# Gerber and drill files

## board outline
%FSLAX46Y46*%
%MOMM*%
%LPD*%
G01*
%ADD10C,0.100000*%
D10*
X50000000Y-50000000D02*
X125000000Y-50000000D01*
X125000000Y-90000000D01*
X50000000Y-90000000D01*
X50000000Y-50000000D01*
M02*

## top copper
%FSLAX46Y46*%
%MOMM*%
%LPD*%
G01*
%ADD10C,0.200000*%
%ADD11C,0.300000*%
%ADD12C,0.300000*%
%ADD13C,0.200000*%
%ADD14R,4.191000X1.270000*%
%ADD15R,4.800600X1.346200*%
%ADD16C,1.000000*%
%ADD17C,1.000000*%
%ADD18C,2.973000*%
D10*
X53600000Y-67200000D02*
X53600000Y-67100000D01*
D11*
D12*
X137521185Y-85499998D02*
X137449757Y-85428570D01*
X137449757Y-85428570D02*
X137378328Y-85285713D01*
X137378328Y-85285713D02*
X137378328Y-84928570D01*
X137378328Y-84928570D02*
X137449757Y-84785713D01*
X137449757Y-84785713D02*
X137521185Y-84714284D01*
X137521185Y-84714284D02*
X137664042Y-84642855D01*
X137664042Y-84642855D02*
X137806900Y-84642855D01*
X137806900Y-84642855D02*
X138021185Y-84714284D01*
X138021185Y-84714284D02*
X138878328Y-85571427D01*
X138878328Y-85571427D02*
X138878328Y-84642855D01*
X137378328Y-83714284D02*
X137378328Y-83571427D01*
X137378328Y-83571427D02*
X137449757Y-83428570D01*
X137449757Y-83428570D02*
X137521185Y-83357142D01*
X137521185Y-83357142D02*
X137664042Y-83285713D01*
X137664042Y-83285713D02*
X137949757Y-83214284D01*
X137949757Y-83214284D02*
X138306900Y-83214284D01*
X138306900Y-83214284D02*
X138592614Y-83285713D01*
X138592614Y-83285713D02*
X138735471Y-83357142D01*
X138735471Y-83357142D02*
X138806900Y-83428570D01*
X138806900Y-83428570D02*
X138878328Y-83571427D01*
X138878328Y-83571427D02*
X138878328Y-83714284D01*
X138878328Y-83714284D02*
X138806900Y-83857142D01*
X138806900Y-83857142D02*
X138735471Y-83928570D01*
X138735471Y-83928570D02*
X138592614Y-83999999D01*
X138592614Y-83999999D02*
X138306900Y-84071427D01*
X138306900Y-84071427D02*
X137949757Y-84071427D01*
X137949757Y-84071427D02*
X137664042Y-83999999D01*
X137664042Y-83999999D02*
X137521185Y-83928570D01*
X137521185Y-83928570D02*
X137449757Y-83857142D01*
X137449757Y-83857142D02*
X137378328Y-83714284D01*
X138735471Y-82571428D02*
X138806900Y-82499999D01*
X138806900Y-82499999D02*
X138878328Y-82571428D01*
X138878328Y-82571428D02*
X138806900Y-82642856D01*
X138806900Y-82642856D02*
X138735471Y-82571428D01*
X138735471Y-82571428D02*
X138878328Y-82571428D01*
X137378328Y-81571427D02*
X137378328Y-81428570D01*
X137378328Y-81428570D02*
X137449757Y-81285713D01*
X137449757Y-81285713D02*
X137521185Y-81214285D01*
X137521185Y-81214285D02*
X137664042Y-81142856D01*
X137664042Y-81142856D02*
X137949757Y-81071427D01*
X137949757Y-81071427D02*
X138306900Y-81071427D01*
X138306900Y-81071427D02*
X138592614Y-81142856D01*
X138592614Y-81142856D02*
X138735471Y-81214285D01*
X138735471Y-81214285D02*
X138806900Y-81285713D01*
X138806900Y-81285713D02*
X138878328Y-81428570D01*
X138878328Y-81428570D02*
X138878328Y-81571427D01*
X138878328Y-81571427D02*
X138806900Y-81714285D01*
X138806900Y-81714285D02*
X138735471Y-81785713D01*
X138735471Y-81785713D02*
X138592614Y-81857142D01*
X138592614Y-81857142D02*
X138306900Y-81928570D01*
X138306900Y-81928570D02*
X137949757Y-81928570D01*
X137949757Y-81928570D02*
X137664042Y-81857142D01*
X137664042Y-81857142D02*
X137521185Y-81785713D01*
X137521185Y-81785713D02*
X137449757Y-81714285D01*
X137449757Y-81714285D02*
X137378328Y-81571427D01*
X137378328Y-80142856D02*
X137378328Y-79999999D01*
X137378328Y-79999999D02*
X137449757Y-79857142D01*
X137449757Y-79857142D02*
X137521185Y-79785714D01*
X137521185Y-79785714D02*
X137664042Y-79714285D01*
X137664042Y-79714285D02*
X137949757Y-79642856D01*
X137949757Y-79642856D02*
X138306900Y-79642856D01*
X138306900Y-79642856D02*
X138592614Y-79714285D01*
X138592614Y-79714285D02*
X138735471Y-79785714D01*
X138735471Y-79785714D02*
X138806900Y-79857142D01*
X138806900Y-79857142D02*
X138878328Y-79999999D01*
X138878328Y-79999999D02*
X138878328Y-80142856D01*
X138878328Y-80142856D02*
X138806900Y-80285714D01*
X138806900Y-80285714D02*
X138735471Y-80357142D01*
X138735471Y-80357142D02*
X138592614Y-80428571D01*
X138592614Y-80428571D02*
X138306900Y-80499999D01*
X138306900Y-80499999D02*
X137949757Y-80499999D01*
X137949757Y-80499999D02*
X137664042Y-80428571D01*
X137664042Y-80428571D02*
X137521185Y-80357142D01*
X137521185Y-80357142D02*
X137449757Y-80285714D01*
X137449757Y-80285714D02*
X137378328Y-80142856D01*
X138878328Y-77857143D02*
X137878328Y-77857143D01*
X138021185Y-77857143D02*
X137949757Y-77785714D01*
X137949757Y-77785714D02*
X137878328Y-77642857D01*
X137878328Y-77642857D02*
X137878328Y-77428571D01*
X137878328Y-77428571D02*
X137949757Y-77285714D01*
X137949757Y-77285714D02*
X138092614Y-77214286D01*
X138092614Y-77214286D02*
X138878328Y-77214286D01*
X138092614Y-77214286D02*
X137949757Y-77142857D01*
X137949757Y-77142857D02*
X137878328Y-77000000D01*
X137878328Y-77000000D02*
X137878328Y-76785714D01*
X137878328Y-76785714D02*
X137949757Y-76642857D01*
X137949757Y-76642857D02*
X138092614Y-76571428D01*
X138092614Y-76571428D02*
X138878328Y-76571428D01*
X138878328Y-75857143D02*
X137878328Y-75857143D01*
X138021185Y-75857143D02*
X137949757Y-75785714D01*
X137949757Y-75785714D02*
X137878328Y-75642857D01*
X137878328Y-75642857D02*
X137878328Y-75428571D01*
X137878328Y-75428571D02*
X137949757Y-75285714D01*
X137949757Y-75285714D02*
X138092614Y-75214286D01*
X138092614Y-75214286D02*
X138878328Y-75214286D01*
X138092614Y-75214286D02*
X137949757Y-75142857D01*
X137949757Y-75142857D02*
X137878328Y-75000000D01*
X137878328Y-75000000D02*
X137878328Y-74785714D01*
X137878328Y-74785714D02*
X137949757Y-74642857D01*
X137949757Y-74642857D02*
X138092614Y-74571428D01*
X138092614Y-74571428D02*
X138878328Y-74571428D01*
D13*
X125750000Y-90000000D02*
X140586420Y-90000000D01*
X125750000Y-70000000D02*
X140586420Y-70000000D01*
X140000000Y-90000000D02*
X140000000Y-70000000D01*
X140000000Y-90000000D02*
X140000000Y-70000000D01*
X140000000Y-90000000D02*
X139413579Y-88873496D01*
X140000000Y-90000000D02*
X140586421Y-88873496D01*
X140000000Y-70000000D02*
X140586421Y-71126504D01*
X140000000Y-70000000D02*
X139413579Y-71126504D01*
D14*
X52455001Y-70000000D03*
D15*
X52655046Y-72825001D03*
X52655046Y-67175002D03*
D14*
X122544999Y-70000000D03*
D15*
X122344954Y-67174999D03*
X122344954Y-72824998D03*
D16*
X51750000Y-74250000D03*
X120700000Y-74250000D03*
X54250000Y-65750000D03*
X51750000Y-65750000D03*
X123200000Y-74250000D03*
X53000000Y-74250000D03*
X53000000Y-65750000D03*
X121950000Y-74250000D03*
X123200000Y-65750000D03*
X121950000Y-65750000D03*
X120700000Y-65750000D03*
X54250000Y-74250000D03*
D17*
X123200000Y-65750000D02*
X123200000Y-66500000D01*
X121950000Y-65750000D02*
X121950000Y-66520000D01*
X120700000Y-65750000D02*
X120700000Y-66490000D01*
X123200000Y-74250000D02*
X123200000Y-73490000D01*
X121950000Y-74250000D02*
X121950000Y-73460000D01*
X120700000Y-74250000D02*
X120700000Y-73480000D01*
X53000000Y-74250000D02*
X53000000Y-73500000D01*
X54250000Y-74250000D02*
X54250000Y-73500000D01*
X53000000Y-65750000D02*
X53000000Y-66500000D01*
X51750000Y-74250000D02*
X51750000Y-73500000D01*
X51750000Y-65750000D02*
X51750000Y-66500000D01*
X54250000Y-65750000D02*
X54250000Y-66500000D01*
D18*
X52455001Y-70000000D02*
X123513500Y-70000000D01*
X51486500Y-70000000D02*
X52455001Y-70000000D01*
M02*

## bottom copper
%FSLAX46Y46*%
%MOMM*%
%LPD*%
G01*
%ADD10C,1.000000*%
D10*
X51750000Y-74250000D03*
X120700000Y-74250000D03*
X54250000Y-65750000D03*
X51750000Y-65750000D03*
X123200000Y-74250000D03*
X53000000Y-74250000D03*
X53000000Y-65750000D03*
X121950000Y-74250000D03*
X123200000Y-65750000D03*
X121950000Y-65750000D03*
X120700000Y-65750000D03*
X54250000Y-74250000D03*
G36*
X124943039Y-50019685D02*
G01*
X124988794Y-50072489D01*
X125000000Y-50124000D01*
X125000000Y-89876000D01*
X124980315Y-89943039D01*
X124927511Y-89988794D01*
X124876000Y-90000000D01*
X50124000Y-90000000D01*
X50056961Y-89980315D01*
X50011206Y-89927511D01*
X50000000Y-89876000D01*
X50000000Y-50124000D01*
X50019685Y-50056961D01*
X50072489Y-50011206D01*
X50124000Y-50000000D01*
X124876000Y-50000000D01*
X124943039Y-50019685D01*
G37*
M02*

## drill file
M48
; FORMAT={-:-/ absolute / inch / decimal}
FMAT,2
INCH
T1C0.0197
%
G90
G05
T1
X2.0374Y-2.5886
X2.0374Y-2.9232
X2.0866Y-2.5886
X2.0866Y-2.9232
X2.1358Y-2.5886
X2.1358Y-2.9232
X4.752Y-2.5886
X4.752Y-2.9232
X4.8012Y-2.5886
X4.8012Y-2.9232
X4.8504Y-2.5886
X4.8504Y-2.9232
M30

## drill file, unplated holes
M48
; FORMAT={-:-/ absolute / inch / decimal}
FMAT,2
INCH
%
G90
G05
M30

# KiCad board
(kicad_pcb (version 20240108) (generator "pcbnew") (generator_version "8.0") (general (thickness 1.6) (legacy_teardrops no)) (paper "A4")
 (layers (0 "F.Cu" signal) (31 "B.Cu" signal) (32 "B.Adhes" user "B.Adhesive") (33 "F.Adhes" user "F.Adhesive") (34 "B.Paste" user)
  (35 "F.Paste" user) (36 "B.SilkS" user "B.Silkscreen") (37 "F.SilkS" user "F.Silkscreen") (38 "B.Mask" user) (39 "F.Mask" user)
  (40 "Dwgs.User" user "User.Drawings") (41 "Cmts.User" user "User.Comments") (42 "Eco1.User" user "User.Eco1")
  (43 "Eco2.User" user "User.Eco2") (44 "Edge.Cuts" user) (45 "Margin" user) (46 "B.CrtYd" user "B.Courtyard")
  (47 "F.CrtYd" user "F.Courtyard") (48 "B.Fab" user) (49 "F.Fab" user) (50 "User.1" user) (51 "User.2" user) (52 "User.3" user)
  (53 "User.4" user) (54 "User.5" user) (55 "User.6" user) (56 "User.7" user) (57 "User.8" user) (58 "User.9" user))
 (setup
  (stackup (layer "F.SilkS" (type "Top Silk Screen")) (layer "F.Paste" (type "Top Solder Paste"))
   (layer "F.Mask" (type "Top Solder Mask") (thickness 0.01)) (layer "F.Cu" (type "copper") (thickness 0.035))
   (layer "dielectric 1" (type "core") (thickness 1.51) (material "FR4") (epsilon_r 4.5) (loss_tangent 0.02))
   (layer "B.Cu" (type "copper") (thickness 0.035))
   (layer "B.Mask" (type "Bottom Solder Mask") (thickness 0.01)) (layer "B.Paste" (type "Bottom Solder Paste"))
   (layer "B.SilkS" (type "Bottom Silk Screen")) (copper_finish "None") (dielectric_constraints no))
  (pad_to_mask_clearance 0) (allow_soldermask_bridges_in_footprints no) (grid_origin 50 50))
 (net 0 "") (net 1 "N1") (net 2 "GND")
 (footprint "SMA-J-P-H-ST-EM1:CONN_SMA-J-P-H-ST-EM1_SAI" (layer "F.Cu") (at 52.16 70 90)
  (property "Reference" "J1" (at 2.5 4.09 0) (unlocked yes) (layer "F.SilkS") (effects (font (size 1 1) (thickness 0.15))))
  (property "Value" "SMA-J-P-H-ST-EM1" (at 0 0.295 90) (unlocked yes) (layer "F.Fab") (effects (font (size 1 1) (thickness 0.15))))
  (pad "1" smd rect (at 0 0.295001 90) (size 1.27 4.191) (layers "F.Cu" "F.Paste" "F.Mask") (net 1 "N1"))
  (pad "2" smd rect (at -2.825001 0.495046 90) (size 1.3462 4.8006) (layers "F.Cu" "F.Paste" "F.Mask") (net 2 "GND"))
  (pad "3" smd rect (at 2.824998 0.495046 90) (size 1.3462 4.8006) (layers "F.Cu" "F.Paste" "F.Mask") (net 2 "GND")))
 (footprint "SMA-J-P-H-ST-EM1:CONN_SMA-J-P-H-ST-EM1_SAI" (layer "F.Cu") (at 122.84 70 -90)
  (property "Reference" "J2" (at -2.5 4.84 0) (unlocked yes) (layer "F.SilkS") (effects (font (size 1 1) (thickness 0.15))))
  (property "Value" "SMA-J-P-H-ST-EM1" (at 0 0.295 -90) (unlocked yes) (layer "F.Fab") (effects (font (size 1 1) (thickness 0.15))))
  (pad "1" smd rect (at 0 0.295001 270) (size 1.27 4.191) (layers "F.Cu" "F.Paste" "F.Mask") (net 1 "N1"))
  (pad "2" smd rect (at -2.825001 0.495046 270) (size 1.3462 4.8006) (layers "F.Cu" "F.Paste" "F.Mask") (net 2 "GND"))
  (pad "3" smd rect (at 2.824998 0.495046 270) (size 1.3462 4.8006) (layers "F.Cu" "F.Paste" "F.Mask") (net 2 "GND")))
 (gr_line (start 53.6 67.2) (end 53.6 67.1) (stroke (width 0.2) (type default)) (layer "F.Cu") (net 2))
 (gr_rect (start 50 50) (end 125 90) (stroke (width 0.1) (type default)) (fill none) (layer "Edge.Cuts"))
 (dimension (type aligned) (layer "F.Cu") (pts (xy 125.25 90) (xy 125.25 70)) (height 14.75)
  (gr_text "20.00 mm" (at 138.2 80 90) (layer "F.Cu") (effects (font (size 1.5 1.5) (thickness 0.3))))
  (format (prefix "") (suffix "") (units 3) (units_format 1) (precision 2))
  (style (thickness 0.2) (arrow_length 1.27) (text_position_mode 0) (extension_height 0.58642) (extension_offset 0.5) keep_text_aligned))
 (segment (start 123.2 65.75) (end 123.2 66.5) (width 1) (layer "F.Cu") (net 2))
 (segment (start 120.7 74.25) (end 120.7 73.48) (width 1) (layer "F.Cu") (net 2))
 (segment (start 53 74.25) (end 53 73.5) (width 1) (layer "F.Cu") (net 2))
 (segment (start 54.25 74.25) (end 54.25 73.5) (width 1) (layer "F.Cu") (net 2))
 (segment (start 53 65.75) (end 53 66.5) (width 1) (layer "F.Cu") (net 2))
 (segment (start 123.2 74.25) (end 123.2 73.49) (width 1) (layer "F.Cu") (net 2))
 (segment (start 121.95 65.75) (end 121.95 66.52) (width 1) (layer "F.Cu") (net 2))
 (segment (start 51.75 74.25) (end 51.75 73.5) (width 1) (layer "F.Cu") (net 2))
 (segment (start 51.75 65.75) (end 51.75 66.5) (width 1) (layer "F.Cu") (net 2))
 (segment (start 54.25 65.75) (end 54.25 66.5) (width 1) (layer "F.Cu") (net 2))
 (segment (start 120.7 65.75) (end 120.7 66.49) (width 1) (layer "F.Cu") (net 2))
 (segment (start 121.95 74.25) (end 121.95 73.46) (width 1) (layer "F.Cu") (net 2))
 (via (at 51.75 74.25) (size 1) (drill 0.5) (layers "F.Cu" "B.Cu") (free yes) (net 2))
 (via (at 120.7 74.25) (size 1) (drill 0.5) (layers "F.Cu" "B.Cu") (free yes) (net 2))
 (via (at 54.25 65.75) (size 1) (drill 0.5) (layers "F.Cu" "B.Cu") (free yes) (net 2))
 (via (at 51.75 65.75) (size 1) (drill 0.5) (layers "F.Cu" "B.Cu") (free yes) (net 2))
 (via (at 123.2 74.25) (size 1) (drill 0.5) (layers "F.Cu" "B.Cu") (free yes) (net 2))
 (via (at 53 74.25) (size 1) (drill 0.5) (layers "F.Cu" "B.Cu") (free yes) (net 2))
 (via (at 53 65.75) (size 1) (drill 0.5) (layers "F.Cu" "B.Cu") (free yes) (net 2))
 (via (at 121.95 74.25) (size 1) (drill 0.5) (layers "F.Cu" "B.Cu") (free yes) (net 2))
 (via (at 123.2 65.75) (size 1) (drill 0.5) (layers "F.Cu" "B.Cu") (free yes) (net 2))
 (via (at 121.95 65.75) (size 1) (drill 0.5) (layers "F.Cu" "B.Cu") (free yes) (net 2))
 (via (at 120.7 65.75) (size 1) (drill 0.5) (layers "F.Cu" "B.Cu") (free yes) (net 2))
 (via (at 54.25 74.25) (size 1) (drill 0.5) (layers "F.Cu" "B.Cu") (free yes) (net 2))
 (segment (start 52.455001 70) (end 123.5135 70) (width 2.973) (layer "F.Cu") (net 1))
 (segment (start 51.4865 70) (end 52.455001 70) (width 2.973) (layer "F.Cu") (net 1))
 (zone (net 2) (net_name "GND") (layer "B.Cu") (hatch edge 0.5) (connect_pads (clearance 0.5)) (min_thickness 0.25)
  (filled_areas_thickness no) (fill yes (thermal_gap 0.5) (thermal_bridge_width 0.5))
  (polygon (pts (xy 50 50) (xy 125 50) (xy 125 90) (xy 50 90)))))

